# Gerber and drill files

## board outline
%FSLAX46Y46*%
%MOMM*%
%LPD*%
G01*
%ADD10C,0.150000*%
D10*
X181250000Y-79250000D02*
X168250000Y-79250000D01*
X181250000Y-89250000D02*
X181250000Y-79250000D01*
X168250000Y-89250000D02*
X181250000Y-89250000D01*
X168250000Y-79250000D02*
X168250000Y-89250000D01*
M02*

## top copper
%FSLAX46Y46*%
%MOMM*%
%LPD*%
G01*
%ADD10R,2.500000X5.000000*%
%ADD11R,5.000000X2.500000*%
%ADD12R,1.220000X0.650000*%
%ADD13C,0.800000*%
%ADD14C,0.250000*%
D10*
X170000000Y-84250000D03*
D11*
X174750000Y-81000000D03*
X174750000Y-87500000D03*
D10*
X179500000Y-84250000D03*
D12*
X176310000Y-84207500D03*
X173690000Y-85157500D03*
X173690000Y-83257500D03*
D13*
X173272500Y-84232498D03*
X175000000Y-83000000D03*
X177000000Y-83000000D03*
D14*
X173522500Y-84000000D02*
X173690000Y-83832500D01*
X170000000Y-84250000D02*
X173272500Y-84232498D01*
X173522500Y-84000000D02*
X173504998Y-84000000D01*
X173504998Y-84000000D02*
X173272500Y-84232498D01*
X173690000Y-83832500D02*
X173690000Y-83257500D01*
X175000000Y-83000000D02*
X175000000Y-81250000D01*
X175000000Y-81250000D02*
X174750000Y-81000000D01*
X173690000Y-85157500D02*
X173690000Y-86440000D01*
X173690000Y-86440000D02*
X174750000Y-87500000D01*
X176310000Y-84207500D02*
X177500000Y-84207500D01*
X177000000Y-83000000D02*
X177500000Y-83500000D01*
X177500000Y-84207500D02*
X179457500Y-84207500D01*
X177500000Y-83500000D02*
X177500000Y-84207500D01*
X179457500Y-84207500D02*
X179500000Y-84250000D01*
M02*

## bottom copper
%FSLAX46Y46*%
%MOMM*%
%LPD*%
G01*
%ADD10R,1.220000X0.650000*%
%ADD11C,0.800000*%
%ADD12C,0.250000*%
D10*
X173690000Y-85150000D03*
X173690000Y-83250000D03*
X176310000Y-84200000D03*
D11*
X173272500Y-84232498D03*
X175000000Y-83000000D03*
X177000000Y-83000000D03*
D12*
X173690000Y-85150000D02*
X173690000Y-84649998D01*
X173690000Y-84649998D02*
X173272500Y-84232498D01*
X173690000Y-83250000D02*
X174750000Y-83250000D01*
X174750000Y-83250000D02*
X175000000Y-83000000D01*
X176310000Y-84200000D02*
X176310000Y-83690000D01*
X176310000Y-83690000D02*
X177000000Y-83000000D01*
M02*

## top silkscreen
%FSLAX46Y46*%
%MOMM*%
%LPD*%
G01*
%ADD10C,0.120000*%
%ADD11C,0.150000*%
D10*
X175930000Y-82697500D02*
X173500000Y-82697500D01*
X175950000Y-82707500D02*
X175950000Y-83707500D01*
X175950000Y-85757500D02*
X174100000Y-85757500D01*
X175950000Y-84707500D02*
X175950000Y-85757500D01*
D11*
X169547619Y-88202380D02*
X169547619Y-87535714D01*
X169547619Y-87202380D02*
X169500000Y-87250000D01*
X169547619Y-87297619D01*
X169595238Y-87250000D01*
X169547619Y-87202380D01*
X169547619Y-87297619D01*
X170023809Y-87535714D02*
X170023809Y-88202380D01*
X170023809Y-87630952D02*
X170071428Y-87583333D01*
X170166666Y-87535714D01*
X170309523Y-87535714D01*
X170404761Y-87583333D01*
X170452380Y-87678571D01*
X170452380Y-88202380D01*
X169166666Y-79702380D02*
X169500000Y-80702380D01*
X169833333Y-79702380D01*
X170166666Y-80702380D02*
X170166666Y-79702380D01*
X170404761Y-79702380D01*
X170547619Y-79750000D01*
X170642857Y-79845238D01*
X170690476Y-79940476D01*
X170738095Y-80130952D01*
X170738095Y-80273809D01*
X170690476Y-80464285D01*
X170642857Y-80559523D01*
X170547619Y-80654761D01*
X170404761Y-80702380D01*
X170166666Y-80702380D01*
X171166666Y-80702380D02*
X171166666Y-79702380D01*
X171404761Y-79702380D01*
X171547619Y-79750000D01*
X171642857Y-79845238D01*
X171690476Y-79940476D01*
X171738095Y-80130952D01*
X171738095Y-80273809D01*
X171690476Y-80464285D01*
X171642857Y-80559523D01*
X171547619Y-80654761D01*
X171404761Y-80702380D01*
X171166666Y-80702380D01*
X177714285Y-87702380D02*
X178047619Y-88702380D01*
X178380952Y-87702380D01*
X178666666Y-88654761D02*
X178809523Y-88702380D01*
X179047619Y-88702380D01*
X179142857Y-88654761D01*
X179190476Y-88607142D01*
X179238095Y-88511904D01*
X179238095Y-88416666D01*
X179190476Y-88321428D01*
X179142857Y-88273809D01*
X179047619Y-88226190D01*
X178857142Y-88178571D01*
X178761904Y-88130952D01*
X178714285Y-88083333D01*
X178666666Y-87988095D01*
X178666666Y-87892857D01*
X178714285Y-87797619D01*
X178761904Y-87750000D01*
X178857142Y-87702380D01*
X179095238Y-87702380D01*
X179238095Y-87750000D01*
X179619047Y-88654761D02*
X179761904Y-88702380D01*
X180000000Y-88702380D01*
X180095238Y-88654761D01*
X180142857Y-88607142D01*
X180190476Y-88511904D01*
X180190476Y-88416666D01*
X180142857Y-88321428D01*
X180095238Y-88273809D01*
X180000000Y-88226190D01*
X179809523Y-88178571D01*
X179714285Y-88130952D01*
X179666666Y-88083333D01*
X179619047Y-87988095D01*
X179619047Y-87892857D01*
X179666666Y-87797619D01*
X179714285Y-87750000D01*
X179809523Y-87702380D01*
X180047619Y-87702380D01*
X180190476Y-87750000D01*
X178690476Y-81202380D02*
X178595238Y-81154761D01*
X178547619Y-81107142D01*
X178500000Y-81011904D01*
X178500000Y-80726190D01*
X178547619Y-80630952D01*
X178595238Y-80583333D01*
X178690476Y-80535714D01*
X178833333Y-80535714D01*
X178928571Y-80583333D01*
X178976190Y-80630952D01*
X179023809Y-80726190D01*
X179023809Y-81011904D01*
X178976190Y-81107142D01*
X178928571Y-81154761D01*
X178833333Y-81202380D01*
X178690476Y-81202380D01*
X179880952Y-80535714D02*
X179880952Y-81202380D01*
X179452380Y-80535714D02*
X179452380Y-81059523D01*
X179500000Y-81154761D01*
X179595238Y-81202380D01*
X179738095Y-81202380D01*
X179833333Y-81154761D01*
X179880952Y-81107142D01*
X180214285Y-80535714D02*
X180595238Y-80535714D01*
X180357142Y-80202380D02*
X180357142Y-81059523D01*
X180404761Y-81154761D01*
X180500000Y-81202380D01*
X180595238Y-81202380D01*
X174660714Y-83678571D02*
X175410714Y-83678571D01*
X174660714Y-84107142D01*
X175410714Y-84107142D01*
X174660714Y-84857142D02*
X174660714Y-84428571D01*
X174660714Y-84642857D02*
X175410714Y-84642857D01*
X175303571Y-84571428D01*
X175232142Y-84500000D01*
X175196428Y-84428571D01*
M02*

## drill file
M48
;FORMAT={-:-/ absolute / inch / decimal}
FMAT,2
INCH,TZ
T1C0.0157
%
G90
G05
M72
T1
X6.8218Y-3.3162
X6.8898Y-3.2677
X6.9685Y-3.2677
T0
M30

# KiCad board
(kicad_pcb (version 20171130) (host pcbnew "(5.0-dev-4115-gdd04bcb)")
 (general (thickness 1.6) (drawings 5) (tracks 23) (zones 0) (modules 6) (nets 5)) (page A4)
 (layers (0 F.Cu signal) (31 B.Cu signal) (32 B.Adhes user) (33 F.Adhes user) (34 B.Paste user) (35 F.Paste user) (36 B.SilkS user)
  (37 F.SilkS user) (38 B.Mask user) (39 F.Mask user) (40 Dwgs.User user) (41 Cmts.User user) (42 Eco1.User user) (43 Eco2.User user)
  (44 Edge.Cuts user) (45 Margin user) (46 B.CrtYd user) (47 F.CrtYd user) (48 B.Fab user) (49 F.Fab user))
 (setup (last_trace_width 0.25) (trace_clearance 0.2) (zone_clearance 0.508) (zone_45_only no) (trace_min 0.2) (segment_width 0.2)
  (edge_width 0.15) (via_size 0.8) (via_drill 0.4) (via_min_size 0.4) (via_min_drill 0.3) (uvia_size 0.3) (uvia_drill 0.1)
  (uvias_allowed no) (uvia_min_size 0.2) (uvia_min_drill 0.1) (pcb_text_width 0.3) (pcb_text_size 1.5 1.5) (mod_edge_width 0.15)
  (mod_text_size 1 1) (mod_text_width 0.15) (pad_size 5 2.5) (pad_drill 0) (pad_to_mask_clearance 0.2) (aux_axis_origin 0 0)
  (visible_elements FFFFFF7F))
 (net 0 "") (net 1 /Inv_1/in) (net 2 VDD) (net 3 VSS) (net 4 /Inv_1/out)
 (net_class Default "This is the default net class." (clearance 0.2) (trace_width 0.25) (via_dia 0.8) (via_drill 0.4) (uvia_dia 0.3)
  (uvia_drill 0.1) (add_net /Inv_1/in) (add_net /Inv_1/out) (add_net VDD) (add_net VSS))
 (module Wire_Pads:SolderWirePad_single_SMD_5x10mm (layer F.Cu) (at 170 84.25 90)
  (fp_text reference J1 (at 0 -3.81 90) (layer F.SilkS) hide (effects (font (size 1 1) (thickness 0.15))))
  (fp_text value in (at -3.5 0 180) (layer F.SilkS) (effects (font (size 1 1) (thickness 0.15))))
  (pad 1 smd rect (at 0 0 90) (size 5 2.5) (layers F.Cu F.Paste F.Mask) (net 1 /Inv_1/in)))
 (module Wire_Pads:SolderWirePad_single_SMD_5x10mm (layer F.Cu) (at 174.75 81)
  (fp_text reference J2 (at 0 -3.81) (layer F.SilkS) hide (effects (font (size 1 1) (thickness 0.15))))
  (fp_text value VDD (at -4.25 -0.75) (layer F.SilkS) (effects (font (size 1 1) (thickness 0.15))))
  (pad 1 smd rect (at 0 0) (size 5 2.5) (layers F.Cu F.Paste F.Mask) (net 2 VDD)))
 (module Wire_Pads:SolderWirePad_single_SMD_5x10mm (layer F.Cu) (at 174.75 87.5)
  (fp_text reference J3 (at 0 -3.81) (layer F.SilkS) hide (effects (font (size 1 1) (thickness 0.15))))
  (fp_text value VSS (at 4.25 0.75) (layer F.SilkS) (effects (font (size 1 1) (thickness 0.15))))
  (pad 1 smd rect (at 0 0) (size 5 2.5) (layers F.Cu F.Paste F.Mask) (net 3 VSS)))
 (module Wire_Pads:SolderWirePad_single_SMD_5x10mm (layer F.Cu) (at 179.5 84.25 90)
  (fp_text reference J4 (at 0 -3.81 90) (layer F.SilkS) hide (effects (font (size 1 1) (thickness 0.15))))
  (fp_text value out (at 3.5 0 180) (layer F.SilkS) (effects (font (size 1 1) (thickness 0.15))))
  (pad 1 smd rect (at 0 0 90) (size 5 2.5) (layers F.Cu F.Paste F.Mask) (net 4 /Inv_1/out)))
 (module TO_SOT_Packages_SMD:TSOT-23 (layer F.Cu) (at 175 84.2075)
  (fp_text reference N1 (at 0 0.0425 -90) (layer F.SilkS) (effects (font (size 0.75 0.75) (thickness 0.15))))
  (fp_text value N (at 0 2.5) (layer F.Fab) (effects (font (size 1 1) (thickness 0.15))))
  (fp_line (start 0.93 -1.51) (end -1.5 -1.51) (layer F.SilkS) (width 0.12))
  (fp_line (start 0.95 -1.5) (end 0.95 -0.5) (layer F.SilkS) (width 0.12))
  (fp_line (start 0.95 1.55) (end -0.9 1.55) (layer F.SilkS) (width 0.12))
  (fp_line (start 0.95 0.5) (end 0.95 1.55) (layer F.SilkS) (width 0.12))
  (pad 3 smd rect (at 1.31 0) (size 1.22 0.65) (layers F.Cu F.Paste F.Mask) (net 4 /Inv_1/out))
  (pad 2 smd rect (at -1.31 0.95) (size 1.22 0.65) (layers F.Cu F.Paste F.Mask) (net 3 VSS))
  (pad 1 smd rect (at -1.31 -0.95) (size 1.22 0.65) (layers F.Cu F.Paste F.Mask) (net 1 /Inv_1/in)))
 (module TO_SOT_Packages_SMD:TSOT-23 (layer B.Cu) (at 175 84.2)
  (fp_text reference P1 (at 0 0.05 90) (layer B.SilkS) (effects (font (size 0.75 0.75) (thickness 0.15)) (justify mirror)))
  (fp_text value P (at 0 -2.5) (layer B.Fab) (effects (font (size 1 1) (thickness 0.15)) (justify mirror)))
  (pad 1 smd rect (at -1.31 0.95) (size 1.22 0.65) (layers B.Cu B.Paste B.Mask) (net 1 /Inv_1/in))
  (pad 2 smd rect (at -1.31 -0.95) (size 1.22 0.65) (layers B.Cu B.Paste B.Mask) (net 2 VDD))
  (pad 3 smd rect (at 1.31 0) (size 1.22 0.65) (layers B.Cu B.Paste B.Mask) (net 4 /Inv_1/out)))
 (gr_line (start 181.25 79.25) (end 168.25 79.25) (layer Edge.Cuts) (width 0.15))
 (gr_line (start 181.25 89.25) (end 181.25 79.25) (layer Edge.Cuts) (width 0.15))
 (gr_line (start 168.25 89.25) (end 181.25 89.25) (layer Edge.Cuts) (width 0.15))
 (gr_line (start 168.25 79.25) (end 168.25 89.25) (layer Edge.Cuts) (width 0.15))
 (segment (start 173.69 85.15) (end 173.69 84.649998) (width 0.25) (layer B.Cu) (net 1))
 (segment (start 173.69 84.649998) (end 173.2725 84.232498) (width 0.25) (layer B.Cu) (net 1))
 (segment (start 173.5225 84) (end 173.69 83.8325) (width 0.25) (layer F.Cu) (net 1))
 (segment (start 170 84.25) (end 173.2725 84.232498) (width 0.25) (layer F.Cu) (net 1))
 (segment (start 173.5225 84) (end 173.504998 84) (width 0.25) (layer F.Cu) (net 1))
 (segment (start 173.504998 84) (end 173.2725 84.232498) (width 0.25) (layer F.Cu) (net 1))
 (via (at 173.2725 84.232498) (size 0.8) (drill 0.4) (layers F.Cu B.Cu) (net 1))
 (segment (start 173.69 83.8325) (end 173.69 83.2575) (width 0.25) (layer F.Cu) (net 1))
 (segment (start 175 83) (end 175 81.25) (width 0.25) (layer F.Cu) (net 2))
 (segment (start 175 81.25) (end 174.75 81) (width 0.25) (layer F.Cu) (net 2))
 (segment (start 173.69 83.25) (end 174.75 83.25) (width 0.25) (layer B.Cu) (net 2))
 (segment (start 174.75 83.25) (end 175 83) (width 0.25) (layer B.Cu) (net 2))
 (via (at 175 83) (size 0.8) (drill 0.4) (layers F.Cu B.Cu) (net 2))
 (segment (start 173.69 85.1575) (end 173.69 86.44) (width 0.25) (layer F.Cu) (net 3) (status 30))
 (segment (start 173.69 86.44) (end 174.75 87.5) (width 0.25) (layer F.Cu) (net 3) (status 30))
 (segment (start 176.31 84.2075) (end 177.5 84.2075) (width 0.25) (layer F.Cu) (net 4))
 (segment (start 177 83) (end 177.5 83.5) (width 0.25) (layer F.Cu) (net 4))
 (segment (start 177.5 84.2075) (end 179.4575 84.2075) (width 0.25) (layer F.Cu) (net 4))
 (segment (start 177.5 83.5) (end 177.5 84.2075) (width 0.25) (layer F.Cu) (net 4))
 (segment (start 176.31 84.2) (end 176.31 83.69) (width 0.25) (layer B.Cu) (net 4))
 (segment (start 176.31 83.69) (end 177 83) (width 0.25) (layer B.Cu) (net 4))
 (via (at 177 83) (size 0.8) (drill 0.4) (layers F.Cu B.Cu) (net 4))
 (segment (start 179.4575 84.2075) (end 179.5 84.25) (width 0.25) (layer F.Cu) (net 4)))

